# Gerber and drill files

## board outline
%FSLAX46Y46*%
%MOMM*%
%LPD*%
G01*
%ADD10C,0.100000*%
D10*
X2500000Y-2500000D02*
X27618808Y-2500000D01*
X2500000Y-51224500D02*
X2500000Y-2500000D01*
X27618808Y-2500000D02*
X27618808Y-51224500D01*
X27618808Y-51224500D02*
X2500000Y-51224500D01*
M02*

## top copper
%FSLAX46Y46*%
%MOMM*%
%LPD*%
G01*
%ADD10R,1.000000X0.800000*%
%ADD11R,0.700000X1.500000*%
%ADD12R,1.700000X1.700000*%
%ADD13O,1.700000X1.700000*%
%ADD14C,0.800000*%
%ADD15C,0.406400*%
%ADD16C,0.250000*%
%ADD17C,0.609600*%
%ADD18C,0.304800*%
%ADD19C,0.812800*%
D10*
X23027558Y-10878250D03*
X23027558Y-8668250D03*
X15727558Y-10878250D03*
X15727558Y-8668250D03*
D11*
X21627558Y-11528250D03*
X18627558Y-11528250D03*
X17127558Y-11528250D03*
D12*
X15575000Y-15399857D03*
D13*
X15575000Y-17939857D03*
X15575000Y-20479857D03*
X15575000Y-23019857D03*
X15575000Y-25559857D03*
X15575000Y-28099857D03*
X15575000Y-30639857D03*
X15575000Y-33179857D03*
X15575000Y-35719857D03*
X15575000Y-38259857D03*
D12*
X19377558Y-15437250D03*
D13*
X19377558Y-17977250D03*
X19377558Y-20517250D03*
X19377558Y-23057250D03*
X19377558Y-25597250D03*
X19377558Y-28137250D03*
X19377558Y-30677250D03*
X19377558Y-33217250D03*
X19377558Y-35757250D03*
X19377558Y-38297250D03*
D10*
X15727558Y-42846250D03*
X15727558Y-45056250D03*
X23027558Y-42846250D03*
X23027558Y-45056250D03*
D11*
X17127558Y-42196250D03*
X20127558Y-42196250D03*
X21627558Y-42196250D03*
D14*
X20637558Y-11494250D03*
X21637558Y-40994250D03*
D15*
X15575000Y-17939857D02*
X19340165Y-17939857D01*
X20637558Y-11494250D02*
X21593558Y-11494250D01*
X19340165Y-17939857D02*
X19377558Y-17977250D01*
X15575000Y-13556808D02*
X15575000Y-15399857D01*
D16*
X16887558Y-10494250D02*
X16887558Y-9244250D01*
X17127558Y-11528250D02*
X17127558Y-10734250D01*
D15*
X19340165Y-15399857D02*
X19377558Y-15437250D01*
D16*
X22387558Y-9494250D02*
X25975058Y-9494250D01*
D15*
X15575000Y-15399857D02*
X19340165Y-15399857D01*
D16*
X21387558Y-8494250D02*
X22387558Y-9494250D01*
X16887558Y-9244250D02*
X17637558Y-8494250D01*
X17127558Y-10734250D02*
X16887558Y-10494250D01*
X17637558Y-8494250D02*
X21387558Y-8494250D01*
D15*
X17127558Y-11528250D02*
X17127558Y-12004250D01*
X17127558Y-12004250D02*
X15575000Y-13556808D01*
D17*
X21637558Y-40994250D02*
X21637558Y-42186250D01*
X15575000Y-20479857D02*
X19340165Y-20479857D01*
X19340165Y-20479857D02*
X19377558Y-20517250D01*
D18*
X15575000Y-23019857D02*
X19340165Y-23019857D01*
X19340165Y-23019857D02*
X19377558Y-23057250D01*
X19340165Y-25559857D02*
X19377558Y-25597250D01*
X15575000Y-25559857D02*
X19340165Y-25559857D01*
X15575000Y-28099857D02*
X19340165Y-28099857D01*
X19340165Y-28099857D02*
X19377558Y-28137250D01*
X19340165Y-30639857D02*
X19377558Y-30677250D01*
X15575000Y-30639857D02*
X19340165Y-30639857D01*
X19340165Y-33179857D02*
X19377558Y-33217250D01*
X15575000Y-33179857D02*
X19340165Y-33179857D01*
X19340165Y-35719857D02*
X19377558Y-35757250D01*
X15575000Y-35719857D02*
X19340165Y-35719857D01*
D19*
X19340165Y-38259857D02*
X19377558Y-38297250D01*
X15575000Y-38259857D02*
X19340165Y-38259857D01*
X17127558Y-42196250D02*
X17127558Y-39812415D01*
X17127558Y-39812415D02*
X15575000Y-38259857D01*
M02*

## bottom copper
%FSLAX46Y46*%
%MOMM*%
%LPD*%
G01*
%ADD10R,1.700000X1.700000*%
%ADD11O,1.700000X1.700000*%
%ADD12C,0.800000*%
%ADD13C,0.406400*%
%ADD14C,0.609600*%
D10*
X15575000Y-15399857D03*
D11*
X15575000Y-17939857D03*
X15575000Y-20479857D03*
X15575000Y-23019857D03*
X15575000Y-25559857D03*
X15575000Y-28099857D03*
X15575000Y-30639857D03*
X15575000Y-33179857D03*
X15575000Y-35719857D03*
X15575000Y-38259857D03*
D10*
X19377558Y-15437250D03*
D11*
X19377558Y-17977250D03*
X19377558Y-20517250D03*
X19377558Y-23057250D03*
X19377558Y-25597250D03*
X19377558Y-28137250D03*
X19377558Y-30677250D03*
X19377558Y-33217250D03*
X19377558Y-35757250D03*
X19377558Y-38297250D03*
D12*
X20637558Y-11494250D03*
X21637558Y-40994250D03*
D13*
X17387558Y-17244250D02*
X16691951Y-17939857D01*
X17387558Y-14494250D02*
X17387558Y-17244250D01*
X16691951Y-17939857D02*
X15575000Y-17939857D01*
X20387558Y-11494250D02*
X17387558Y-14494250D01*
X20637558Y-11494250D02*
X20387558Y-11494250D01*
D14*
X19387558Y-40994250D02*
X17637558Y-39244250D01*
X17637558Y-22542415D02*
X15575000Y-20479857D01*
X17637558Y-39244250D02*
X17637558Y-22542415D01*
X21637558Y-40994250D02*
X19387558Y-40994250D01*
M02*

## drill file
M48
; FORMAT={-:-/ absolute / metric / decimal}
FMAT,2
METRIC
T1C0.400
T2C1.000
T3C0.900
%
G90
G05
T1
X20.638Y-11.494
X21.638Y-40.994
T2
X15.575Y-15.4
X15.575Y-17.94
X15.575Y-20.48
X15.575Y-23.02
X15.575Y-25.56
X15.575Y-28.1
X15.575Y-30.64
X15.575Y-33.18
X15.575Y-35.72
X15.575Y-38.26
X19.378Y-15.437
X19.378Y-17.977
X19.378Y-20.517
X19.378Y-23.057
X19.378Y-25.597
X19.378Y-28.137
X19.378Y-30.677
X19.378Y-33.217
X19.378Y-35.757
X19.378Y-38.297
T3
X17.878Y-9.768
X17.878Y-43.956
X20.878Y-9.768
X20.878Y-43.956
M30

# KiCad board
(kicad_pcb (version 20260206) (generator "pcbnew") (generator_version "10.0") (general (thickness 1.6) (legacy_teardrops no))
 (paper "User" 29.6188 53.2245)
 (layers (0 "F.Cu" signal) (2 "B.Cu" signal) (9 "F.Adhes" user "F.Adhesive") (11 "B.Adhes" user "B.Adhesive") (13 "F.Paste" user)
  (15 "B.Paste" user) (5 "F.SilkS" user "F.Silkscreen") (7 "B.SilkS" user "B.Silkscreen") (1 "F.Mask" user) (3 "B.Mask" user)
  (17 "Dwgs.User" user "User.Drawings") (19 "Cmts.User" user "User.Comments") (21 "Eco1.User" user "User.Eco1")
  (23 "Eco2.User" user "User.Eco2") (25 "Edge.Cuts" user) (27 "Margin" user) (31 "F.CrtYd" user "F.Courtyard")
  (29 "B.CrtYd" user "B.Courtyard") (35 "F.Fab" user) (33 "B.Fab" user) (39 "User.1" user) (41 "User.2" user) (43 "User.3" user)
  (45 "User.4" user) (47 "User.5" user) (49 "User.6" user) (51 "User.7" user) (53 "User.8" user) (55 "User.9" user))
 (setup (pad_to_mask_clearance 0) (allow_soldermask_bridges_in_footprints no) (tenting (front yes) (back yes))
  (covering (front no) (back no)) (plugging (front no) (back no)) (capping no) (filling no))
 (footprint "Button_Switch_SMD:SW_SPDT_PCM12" (layer "F.Cu") (at 19.377558 10.09825 180)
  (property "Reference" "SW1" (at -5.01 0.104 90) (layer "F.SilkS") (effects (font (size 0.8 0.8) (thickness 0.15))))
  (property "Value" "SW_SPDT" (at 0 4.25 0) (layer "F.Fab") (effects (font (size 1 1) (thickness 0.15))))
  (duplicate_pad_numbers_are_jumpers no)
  (pad "" smd rect (at -3.65 -0.78 180) (size 1 0.8) (layers "F.Cu" "F.Mask" "F.Paste"))
  (pad "" smd rect (at -3.65 1.43 180) (size 1 0.8) (layers "F.Cu" "F.Mask" "F.Paste"))
  (pad "" np_thru_hole circle (at -1.5 0.33 180) (size 0.9 0.9) (drill 0.9) (layers "*.Cu" "*.Mask"))
  (pad "" np_thru_hole circle (at 1.5 0.33 180) (size 0.9 0.9) (drill 0.9) (layers "*.Cu" "*.Mask"))
  (pad "" smd rect (at 3.65 -0.78 180) (size 1 0.8) (layers "F.Cu" "F.Mask" "F.Paste"))
  (pad "" smd rect (at 3.65 1.43 180) (size 1 0.8) (layers "F.Cu" "F.Mask" "F.Paste"))
  (pad "1" smd rect (at -2.25 -1.43 180) (size 0.7 1.5) (layers "F.Cu" "F.Mask" "F.Paste") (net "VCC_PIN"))
  (pad "2" smd rect (at 0.75 -1.43 180) (size 0.7 1.5) (layers "F.Cu" "F.Mask" "F.Paste") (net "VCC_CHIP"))
  (pad "3" smd rect (at 2.25 -1.43 180) (size 0.7 1.5) (layers "F.Cu" "F.Mask" "F.Paste") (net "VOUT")))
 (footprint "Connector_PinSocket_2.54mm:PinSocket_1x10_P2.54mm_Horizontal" (layer "F.Cu") (at 15.575 15.399857)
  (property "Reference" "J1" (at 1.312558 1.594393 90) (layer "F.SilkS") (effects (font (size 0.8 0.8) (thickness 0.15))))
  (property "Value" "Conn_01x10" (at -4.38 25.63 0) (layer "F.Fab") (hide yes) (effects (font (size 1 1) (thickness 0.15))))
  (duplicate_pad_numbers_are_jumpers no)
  (pad "1" thru_hole rect (at 0 0) (size 1.7 1.7) (drill 1) (layers "*.Cu" "*.Mask") (remove_unused_layers no) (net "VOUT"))
  (pad "2" thru_hole oval (at 0 2.54) (size 1.7 1.7) (drill 1) (layers "*.Cu" "*.Mask") (remove_unused_layers no) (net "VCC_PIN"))
  (pad "3" thru_hole oval (at 0 5.08) (size 1.7 1.7) (drill 1) (layers "*.Cu" "*.Mask") (remove_unused_layers no) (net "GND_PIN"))
  (pad "4" thru_hole oval (at 0 7.62) (size 1.7 1.7) (drill 1) (layers "*.Cu" "*.Mask") (remove_unused_layers no) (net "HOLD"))
  (pad "5" thru_hole oval (at 0 10.16) (size 1.7 1.7) (drill 1) (layers "*.Cu" "*.Mask") (remove_unused_layers no) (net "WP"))
  (pad "6" thru_hole oval (at 0 12.7) (size 1.7 1.7) (drill 1) (layers "*.Cu" "*.Mask") (remove_unused_layers no) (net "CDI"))
  (pad "7" thru_hole oval (at 0 15.24) (size 1.7 1.7) (drill 1) (layers "*.Cu" "*.Mask") (remove_unused_layers no) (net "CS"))
  (pad "8" thru_hole oval (at 0 17.78) (size 1.7 1.7) (drill 1) (layers "*.Cu" "*.Mask") (remove_unused_layers no) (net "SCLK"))
  (pad "9" thru_hole oval (at 0 20.32) (size 1.7 1.7) (drill 1) (layers "*.Cu" "*.Mask") (remove_unused_layers no) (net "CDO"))
  (pad "10" thru_hole oval (at 0 22.86) (size 1.7 1.7) (drill 1) (layers "*.Cu" "*.Mask") (remove_unused_layers no) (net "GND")))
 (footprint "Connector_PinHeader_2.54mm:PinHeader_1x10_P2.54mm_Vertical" (layer "F.Cu") (at 19.377558 15.43725)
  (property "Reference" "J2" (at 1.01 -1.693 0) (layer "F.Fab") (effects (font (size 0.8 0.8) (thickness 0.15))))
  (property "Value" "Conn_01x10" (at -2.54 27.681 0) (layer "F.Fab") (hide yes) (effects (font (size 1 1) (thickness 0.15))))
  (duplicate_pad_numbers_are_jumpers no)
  (pad "1" thru_hole rect (at 0 0) (size 1.7 1.7) (drill 1) (layers "*.Cu" "*.Mask") (remove_unused_layers no) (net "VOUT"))
  (pad "2" thru_hole oval (at 0 2.54) (size 1.7 1.7) (drill 1) (layers "*.Cu" "*.Mask") (remove_unused_layers no) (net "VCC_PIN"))
  (pad "3" thru_hole oval (at 0 5.08) (size 1.7 1.7) (drill 1) (layers "*.Cu" "*.Mask") (remove_unused_layers no) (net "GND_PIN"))
  (pad "4" thru_hole oval (at 0 7.62) (size 1.7 1.7) (drill 1) (layers "*.Cu" "*.Mask") (remove_unused_layers no) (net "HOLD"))
  (pad "5" thru_hole oval (at 0 10.16) (size 1.7 1.7) (drill 1) (layers "*.Cu" "*.Mask") (remove_unused_layers no) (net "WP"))
  (pad "6" thru_hole oval (at 0 12.7) (size 1.7 1.7) (drill 1) (layers "*.Cu" "*.Mask") (remove_unused_layers no) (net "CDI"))
  (pad "7" thru_hole oval (at 0 15.24) (size 1.7 1.7) (drill 1) (layers "*.Cu" "*.Mask") (remove_unused_layers no) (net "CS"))
  (pad "8" thru_hole oval (at 0 17.78) (size 1.7 1.7) (drill 1) (layers "*.Cu" "*.Mask") (remove_unused_layers no) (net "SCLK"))
  (pad "9" thru_hole oval (at 0 20.32) (size 1.7 1.7) (drill 1) (layers "*.Cu" "*.Mask") (remove_unused_layers no) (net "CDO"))
  (pad "10" thru_hole oval (at 0 22.86) (size 1.7 1.7) (drill 1) (layers "*.Cu" "*.Mask") (remove_unused_layers no) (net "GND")))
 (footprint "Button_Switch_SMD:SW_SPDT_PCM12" (layer "F.Cu") (at 19.377558 43.62625)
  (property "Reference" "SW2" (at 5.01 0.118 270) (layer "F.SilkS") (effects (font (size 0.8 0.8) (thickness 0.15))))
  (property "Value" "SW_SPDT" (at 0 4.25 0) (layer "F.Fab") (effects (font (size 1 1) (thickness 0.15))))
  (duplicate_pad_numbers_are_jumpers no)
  (pad "" smd rect (at -3.65 -0.78) (size 1 0.8) (layers "F.Cu" "F.Mask" "F.Paste"))
  (pad "" smd rect (at -3.65 1.43) (size 1 0.8) (layers "F.Cu" "F.Mask" "F.Paste"))
  (pad "" np_thru_hole circle (at -1.5 0.33) (size 0.9 0.9) (drill 0.9) (layers "*.Cu" "*.Mask"))
  (pad "" np_thru_hole circle (at 1.5 0.33) (size 0.9 0.9) (drill 0.9) (layers "*.Cu" "*.Mask"))
  (pad "" smd rect (at 3.65 -0.78) (size 1 0.8) (layers "F.Cu" "F.Mask" "F.Paste"))
  (pad "" smd rect (at 3.65 1.43) (size 1 0.8) (layers "F.Cu" "F.Mask" "F.Paste"))
  (pad "1" smd rect (at -2.25 -1.43) (size 0.7 1.5) (layers "F.Cu" "F.Mask" "F.Paste") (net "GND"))
  (pad "2" smd rect (at 0.75 -1.43) (size 0.7 1.5) (layers "F.Cu" "F.Mask" "F.Paste") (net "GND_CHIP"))
  (pad "3" smd rect (at 2.25 -1.43) (size 0.7 1.5) (layers "F.Cu" "F.Mask" "F.Paste") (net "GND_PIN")))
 (gr_line (start 2.5 2.5) (end 27.618808 2.5) (stroke (width 0.1) (type default)) (layer "Edge.Cuts"))
 (gr_line (start 2.5 51.2245) (end 2.5 2.5) (stroke (width 0.1) (type default)) (layer "Edge.Cuts"))
 (gr_line (start 27.618808 2.5) (end 27.618808 51.2245) (stroke (width 0.1) (type default)) (layer "Edge.Cuts"))
 (gr_line (start 27.618808 51.2245) (end 2.5 51.2245) (stroke (width 0.1) (type default)) (layer "Edge.Cuts"))
 (segment (start 15.575 17.939857) (end 19.340165 17.939857) (width 0.4064) (layer "F.Cu") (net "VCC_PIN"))
 (segment (start 20.637558 11.49425) (end 21.593558 11.49425) (width 0.4064) (layer "F.Cu") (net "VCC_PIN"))
 (segment (start 19.340165 17.939857) (end 19.377558 17.97725) (width 0.4064) (layer "F.Cu") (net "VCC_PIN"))
 (via (at 20.637558 11.49425) (size 0.8) (drill 0.4) (layers "F.Cu" "B.Cu") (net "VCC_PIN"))
 (segment (start 17.387558 17.24425) (end 16.691951 17.939857) (width 0.4064) (layer "B.Cu") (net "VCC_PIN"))
 (segment (start 17.387558 14.49425) (end 17.387558 17.24425) (width 0.4064) (layer "B.Cu") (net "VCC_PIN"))
 (segment (start 16.691951 17.939857) (end 15.575 17.939857) (width 0.4064) (layer "B.Cu") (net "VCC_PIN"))
 (segment (start 20.387558 11.49425) (end 17.387558 14.49425) (width 0.4064) (layer "B.Cu") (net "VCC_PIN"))
 (segment (start 20.637558 11.49425) (end 20.387558 11.49425) (width 0.4064) (layer "B.Cu") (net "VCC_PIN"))
 (segment (start 15.575 13.556808) (end 15.575 15.399857) (width 0.4064) (layer "F.Cu") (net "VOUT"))
 (segment (start 16.887558 10.49425) (end 16.887558 9.24425) (width 0.25) (layer "F.Cu") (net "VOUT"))
 (segment (start 17.127558 11.52825) (end 17.127558 10.73425) (width 0.25) (layer "F.Cu") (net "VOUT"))
 (segment (start 19.340165 15.399857) (end 19.377558 15.43725) (width 0.4064) (layer "F.Cu") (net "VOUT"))
 (segment (start 22.387558 9.49425) (end 25.975058 9.49425) (width 0.25) (layer "F.Cu") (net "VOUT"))
 (segment (start 15.575 15.399857) (end 19.340165 15.399857) (width 0.4064) (layer "F.Cu") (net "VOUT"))
 (segment (start 21.387558 8.49425) (end 22.387558 9.49425) (width 0.25) (layer "F.Cu") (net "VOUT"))
 (segment (start 16.887558 9.24425) (end 17.637558 8.49425) (width 0.25) (layer "F.Cu") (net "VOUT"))
 (segment (start 17.127558 10.73425) (end 16.887558 10.49425) (width 0.25) (layer "F.Cu") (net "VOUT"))
 (segment (start 17.637558 8.49425) (end 21.387558 8.49425) (width 0.25) (layer "F.Cu") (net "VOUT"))
 (segment (start 17.127558 11.52825) (end 17.127558 12.00425) (width 0.4064) (layer "F.Cu") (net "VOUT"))
 (segment (start 17.127558 12.00425) (end 15.575 13.556808) (width 0.4064) (layer "F.Cu") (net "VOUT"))
 (segment (start 21.637558 40.99425) (end 21.637558 42.18625) (width 0.6096) (layer "F.Cu") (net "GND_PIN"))
 (segment (start 15.575 20.479857) (end 19.340165 20.479857) (width 0.6096) (layer "F.Cu") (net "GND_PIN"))
 (segment (start 19.340165 20.479857) (end 19.377558 20.51725) (width 0.6096) (layer "F.Cu") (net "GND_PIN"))
 (via (at 21.637558 40.99425) (size 0.8) (drill 0.4) (layers "F.Cu" "B.Cu") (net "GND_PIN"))
 (segment (start 19.387558 40.99425) (end 17.637558 39.24425) (width 0.6096) (layer "B.Cu") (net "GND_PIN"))
 (segment (start 17.637558 22.542415) (end 15.575 20.479857) (width 0.6096) (layer "B.Cu") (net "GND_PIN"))
 (segment (start 17.637558 39.24425) (end 17.637558 22.542415) (width 0.6096) (layer "B.Cu") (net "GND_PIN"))
 (segment (start 21.637558 40.99425) (end 19.387558 40.99425) (width 0.6096) (layer "B.Cu") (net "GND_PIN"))
 (segment (start 15.575 23.019857) (end 19.340165 23.019857) (width 0.3048) (layer "F.Cu") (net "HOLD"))
 (segment (start 19.340165 23.019857) (end 19.377558 23.05725) (width 0.3048) (layer "F.Cu") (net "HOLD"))
 (segment (start 19.340165 25.559857) (end 19.377558 25.59725) (width 0.3048) (layer "F.Cu") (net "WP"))
 (segment (start 15.575 25.559857) (end 19.340165 25.559857) (width 0.3048) (layer "F.Cu") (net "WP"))
 (segment (start 15.575 28.099857) (end 19.340165 28.099857) (width 0.3048) (layer "F.Cu") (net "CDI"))
 (segment (start 19.340165 28.099857) (end 19.377558 28.13725) (width 0.3048) (layer "F.Cu") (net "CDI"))
 (segment (start 19.340165 30.639857) (end 19.377558 30.67725) (width 0.3048) (layer "F.Cu") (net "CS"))
 (segment (start 15.575 30.639857) (end 19.340165 30.639857) (width 0.3048) (layer "F.Cu") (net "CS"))
 (segment (start 19.340165 33.179857) (end 19.377558 33.21725) (width 0.3048) (layer "F.Cu") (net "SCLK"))
 (segment (start 15.575 33.179857) (end 19.340165 33.179857) (width 0.3048) (layer "F.Cu") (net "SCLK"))
 (segment (start 19.340165 35.719857) (end 19.377558 35.75725) (width 0.3048) (layer "F.Cu") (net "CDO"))
 (segment (start 15.575 35.719857) (end 19.340165 35.719857) (width 0.3048) (layer "F.Cu") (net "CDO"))
 (segment (start 19.340165 38.259857) (end 19.377558 38.29725) (width 0.8128) (layer "F.Cu") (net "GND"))
 (segment (start 15.575 38.259857) (end 19.340165 38.259857) (width 0.8128) (layer "F.Cu") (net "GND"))
 (segment (start 17.127558 42.19625) (end 17.127558 39.812415) (width 0.8128) (layer "F.Cu") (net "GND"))
 (segment (start 17.127558 39.812415) (end 15.575 38.259857) (width 0.8128) (layer "F.Cu") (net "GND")))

